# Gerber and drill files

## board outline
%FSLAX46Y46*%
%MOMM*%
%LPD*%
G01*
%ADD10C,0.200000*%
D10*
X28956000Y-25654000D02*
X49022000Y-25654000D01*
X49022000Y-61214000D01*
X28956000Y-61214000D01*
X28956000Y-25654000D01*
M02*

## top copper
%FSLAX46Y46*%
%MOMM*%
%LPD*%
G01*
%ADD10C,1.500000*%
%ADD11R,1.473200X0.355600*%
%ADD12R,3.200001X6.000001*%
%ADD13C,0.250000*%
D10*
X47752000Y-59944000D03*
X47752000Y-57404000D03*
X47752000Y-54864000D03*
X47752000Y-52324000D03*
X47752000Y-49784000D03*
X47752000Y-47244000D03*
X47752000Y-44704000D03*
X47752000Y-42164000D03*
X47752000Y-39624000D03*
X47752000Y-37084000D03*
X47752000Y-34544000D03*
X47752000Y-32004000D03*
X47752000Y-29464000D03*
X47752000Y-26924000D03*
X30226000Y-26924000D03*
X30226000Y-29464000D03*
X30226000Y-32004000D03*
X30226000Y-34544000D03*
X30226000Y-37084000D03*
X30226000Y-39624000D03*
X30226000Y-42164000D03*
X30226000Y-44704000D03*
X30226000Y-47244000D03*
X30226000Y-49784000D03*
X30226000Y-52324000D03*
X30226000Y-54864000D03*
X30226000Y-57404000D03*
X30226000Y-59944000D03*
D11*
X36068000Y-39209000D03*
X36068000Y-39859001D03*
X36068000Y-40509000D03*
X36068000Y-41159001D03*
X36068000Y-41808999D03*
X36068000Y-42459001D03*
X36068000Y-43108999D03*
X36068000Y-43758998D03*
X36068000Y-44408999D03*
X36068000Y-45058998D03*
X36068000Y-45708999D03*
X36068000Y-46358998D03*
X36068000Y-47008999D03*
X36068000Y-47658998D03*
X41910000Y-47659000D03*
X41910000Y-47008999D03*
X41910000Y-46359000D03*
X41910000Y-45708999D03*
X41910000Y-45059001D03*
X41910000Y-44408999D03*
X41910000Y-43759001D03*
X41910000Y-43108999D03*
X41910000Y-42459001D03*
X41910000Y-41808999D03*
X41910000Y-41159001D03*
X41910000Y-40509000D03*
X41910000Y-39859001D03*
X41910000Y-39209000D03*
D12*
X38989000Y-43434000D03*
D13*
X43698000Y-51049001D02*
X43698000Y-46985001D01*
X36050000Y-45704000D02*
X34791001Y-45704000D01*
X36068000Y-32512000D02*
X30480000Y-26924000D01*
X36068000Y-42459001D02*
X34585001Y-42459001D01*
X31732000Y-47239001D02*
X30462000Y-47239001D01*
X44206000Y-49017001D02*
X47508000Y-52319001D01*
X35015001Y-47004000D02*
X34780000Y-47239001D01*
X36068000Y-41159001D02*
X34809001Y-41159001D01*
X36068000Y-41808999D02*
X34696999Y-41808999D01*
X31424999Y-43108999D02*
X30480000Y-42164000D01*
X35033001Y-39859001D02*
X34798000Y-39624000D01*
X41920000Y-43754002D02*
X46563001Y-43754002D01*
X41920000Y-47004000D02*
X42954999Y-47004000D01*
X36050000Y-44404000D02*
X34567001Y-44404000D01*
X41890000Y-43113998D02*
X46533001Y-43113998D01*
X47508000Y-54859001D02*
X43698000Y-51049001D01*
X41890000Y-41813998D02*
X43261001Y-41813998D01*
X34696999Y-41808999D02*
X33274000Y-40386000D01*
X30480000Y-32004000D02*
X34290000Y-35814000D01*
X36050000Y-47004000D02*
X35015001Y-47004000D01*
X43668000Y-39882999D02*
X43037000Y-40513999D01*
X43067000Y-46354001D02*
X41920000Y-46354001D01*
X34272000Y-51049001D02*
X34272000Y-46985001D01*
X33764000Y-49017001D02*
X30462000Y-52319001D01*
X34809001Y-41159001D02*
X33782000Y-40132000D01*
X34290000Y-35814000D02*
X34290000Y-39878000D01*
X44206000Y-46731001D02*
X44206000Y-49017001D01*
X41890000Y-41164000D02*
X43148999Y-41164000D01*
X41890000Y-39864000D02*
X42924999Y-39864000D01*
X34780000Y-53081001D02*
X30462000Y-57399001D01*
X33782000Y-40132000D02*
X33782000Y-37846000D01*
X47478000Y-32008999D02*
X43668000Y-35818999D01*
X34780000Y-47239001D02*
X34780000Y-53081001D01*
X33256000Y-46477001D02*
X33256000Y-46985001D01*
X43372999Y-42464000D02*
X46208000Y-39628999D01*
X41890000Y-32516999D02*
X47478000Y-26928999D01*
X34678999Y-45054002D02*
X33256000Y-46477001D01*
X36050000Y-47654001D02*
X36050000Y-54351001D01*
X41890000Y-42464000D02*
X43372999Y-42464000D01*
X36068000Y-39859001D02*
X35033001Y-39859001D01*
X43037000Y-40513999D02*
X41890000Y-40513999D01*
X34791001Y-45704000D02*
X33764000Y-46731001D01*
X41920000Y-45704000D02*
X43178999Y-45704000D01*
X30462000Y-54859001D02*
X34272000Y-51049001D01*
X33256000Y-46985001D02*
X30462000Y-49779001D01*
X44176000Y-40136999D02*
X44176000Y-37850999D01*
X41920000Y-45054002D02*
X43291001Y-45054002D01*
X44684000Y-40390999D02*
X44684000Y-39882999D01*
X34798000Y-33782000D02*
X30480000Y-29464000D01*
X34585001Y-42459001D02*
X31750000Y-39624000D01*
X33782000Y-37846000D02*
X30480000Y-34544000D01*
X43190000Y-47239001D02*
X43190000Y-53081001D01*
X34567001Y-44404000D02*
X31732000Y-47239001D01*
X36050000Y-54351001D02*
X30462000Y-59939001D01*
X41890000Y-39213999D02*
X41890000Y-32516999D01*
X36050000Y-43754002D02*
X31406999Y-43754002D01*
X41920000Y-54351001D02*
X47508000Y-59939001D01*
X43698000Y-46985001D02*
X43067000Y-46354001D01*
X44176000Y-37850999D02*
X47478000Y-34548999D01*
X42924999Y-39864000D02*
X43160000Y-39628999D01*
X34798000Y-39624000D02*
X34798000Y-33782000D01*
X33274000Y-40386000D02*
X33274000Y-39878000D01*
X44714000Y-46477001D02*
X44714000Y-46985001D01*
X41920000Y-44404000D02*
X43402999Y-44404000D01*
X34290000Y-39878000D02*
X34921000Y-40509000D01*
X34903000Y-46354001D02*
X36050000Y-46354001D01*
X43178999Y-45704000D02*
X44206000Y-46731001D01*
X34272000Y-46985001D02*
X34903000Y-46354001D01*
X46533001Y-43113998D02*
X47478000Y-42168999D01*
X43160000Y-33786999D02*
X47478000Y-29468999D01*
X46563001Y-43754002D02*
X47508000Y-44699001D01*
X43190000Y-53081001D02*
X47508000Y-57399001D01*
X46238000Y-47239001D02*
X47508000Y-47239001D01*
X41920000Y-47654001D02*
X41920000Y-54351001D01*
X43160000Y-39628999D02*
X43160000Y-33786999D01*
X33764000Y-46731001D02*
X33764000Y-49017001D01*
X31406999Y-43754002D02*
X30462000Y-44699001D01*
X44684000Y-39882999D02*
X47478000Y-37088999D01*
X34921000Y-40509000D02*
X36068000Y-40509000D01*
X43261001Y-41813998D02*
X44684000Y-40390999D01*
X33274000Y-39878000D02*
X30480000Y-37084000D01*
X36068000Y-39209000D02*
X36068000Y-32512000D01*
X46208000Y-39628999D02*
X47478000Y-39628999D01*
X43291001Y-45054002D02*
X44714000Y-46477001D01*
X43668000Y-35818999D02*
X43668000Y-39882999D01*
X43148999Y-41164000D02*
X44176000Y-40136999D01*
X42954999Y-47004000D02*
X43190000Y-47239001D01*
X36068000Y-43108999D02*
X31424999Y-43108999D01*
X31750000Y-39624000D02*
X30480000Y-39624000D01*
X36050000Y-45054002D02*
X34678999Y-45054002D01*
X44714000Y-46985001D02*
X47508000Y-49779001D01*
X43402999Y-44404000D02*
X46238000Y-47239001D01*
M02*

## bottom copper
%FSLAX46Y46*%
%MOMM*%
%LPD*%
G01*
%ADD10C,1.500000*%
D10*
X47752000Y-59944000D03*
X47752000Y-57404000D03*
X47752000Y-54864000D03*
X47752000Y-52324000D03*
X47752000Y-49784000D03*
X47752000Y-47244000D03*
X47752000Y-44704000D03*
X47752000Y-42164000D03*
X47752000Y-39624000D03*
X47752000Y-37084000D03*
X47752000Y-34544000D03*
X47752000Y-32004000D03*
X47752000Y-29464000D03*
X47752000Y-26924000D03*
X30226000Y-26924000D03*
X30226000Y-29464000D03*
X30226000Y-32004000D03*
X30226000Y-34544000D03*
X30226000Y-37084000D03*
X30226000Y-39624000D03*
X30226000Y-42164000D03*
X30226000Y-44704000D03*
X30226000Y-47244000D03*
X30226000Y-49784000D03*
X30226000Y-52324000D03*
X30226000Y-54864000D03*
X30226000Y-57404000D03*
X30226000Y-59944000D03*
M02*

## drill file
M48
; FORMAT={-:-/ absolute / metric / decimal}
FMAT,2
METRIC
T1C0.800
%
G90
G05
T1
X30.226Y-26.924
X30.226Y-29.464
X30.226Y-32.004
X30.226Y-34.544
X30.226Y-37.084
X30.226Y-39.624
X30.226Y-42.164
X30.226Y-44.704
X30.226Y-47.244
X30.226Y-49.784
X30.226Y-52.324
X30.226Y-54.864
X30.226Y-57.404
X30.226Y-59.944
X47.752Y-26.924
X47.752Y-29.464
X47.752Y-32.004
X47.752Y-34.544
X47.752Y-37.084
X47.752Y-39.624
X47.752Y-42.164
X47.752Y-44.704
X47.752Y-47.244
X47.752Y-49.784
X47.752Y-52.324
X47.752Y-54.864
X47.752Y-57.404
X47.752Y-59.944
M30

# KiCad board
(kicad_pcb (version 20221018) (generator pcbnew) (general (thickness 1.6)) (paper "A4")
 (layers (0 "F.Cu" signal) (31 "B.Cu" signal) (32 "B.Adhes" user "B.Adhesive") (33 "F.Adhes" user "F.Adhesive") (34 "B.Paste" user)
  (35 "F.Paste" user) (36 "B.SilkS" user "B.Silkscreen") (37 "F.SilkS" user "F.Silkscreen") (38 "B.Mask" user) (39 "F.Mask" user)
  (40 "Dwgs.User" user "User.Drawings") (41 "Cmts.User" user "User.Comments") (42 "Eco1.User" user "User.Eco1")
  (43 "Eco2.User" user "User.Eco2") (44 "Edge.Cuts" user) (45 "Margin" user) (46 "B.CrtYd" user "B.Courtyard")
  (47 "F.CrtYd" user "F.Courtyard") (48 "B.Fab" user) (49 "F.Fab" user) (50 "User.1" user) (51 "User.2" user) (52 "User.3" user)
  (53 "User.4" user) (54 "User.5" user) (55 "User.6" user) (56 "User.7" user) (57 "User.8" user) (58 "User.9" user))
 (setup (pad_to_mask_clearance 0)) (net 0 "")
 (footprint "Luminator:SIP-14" (layer "F.Cu") (at 47.752 43.434 90)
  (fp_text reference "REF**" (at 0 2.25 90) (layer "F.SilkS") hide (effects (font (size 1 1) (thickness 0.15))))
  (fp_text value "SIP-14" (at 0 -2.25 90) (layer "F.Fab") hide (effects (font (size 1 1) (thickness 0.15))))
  (pad "1" thru_hole circle (at -16.51 0 90) (size 1.5 1.5) (drill 0.8) (layers "*.Cu" "*.Mask"))
  (pad "2" thru_hole circle (at -13.97 0 90) (size 1.5 1.5) (drill 0.8) (layers "*.Cu" "*.Mask"))
  (pad "3" thru_hole circle (at -11.43 0 90) (size 1.5 1.5) (drill 0.8) (layers "*.Cu" "*.Mask"))
  (pad "4" thru_hole circle (at -8.89 0 90) (size 1.5 1.5) (drill 0.8) (layers "*.Cu" "*.Mask"))
  (pad "5" thru_hole circle (at -6.35 0 90) (size 1.5 1.5) (drill 0.8) (layers "*.Cu" "*.Mask"))
  (pad "6" thru_hole circle (at -3.81 0 90) (size 1.5 1.5) (drill 0.8) (layers "*.Cu" "*.Mask"))
  (pad "7" thru_hole circle (at -1.27 0 90) (size 1.5 1.5) (drill 0.8) (layers "*.Cu" "*.Mask"))
  (pad "8" thru_hole circle (at 1.27 0 90) (size 1.5 1.5) (drill 0.8) (layers "*.Cu" "*.Mask"))
  (pad "9" thru_hole circle (at 3.81 0 90) (size 1.5 1.5) (drill 0.8) (layers "*.Cu" "*.Mask"))
  (pad "10" thru_hole circle (at 6.35 0 90) (size 1.5 1.5) (drill 0.8) (layers "*.Cu" "*.Mask"))
  (pad "11" thru_hole circle (at 8.89 0 90) (size 1.5 1.5) (drill 0.8) (layers "*.Cu" "*.Mask"))
  (pad "12" thru_hole circle (at 11.43 0 90) (size 1.5 1.5) (drill 0.8) (layers "*.Cu" "*.Mask"))
  (pad "13" thru_hole circle (at 13.97 0 90) (size 1.5 1.5) (drill 0.8) (layers "*.Cu" "*.Mask"))
  (pad "14" thru_hole circle (at 16.51 0 90) (size 1.5 1.5) (drill 0.8) (layers "*.Cu" "*.Mask")))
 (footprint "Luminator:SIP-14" (layer "F.Cu") (at 30.226 43.434 -90)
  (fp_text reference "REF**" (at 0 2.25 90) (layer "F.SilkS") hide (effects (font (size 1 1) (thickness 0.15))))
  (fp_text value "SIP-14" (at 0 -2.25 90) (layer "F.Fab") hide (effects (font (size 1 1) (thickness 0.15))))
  (pad "1" thru_hole circle (at -16.51 0 270) (size 1.5 1.5) (drill 0.8) (layers "*.Cu" "*.Mask"))
  (pad "2" thru_hole circle (at -13.97 0 270) (size 1.5 1.5) (drill 0.8) (layers "*.Cu" "*.Mask"))
  (pad "3" thru_hole circle (at -11.43 0 270) (size 1.5 1.5) (drill 0.8) (layers "*.Cu" "*.Mask"))
  (pad "4" thru_hole circle (at -8.89 0 270) (size 1.5 1.5) (drill 0.8) (layers "*.Cu" "*.Mask"))
  (pad "5" thru_hole circle (at -6.35 0 270) (size 1.5 1.5) (drill 0.8) (layers "*.Cu" "*.Mask"))
  (pad "6" thru_hole circle (at -3.81 0 270) (size 1.5 1.5) (drill 0.8) (layers "*.Cu" "*.Mask"))
  (pad "7" thru_hole circle (at -1.27 0 270) (size 1.5 1.5) (drill 0.8) (layers "*.Cu" "*.Mask"))
  (pad "8" thru_hole circle (at 1.27 0 270) (size 1.5 1.5) (drill 0.8) (layers "*.Cu" "*.Mask"))
  (pad "9" thru_hole circle (at 3.81 0 270) (size 1.5 1.5) (drill 0.8) (layers "*.Cu" "*.Mask"))
  (pad "10" thru_hole circle (at 6.35 0 270) (size 1.5 1.5) (drill 0.8) (layers "*.Cu" "*.Mask"))
  (pad "11" thru_hole circle (at 8.89 0 270) (size 1.5 1.5) (drill 0.8) (layers "*.Cu" "*.Mask"))
  (pad "12" thru_hole circle (at 11.43 0 270) (size 1.5 1.5) (drill 0.8) (layers "*.Cu" "*.Mask"))
  (pad "13" thru_hole circle (at 13.97 0 270) (size 1.5 1.5) (drill 0.8) (layers "*.Cu" "*.Mask"))
  (pad "14" thru_hole circle (at 16.51 0 270) (size 1.5 1.5) (drill 0.8) (layers "*.Cu" "*.Mask")))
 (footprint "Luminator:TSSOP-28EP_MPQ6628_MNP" (layer "F.Cu") (at 38.989 43.434)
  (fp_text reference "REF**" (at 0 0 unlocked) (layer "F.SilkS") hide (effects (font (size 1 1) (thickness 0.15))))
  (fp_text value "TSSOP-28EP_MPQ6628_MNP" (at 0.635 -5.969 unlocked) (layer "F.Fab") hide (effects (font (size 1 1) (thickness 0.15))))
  (pad "1" smd rect (at -2.921 -4.225) (size 1.4732 0.3556) (layers "F.Cu" "F.Paste" "F.Mask"))
  (pad "2" smd rect (at -2.921 -3.574999) (size 1.4732 0.3556) (layers "F.Cu" "F.Paste" "F.Mask"))
  (pad "3" smd rect (at -2.921 -2.925) (size 1.4732 0.3556) (layers "F.Cu" "F.Paste" "F.Mask"))
  (pad "4" smd rect (at -2.921 -2.274999) (size 1.4732 0.3556) (layers "F.Cu" "F.Paste" "F.Mask"))
  (pad "5" smd rect (at -2.921 -1.625001) (size 1.4732 0.3556) (layers "F.Cu" "F.Paste" "F.Mask"))
  (pad "6" smd rect (at -2.921 -0.974999) (size 1.4732 0.3556) (layers "F.Cu" "F.Paste" "F.Mask"))
  (pad "7" smd rect (at -2.921 -0.325001) (size 1.4732 0.3556) (layers "F.Cu" "F.Paste" "F.Mask"))
  (pad "8" smd rect (at -2.921 0.324998) (size 1.4732 0.3556) (layers "F.Cu" "F.Paste" "F.Mask"))
  (pad "9" smd rect (at -2.921 0.974999) (size 1.4732 0.3556) (layers "F.Cu" "F.Paste" "F.Mask"))
  (pad "10" smd rect (at -2.921 1.624998) (size 1.4732 0.3556) (layers "F.Cu" "F.Paste" "F.Mask"))
  (pad "11" smd rect (at -2.921 2.274999) (size 1.4732 0.3556) (layers "F.Cu" "F.Paste" "F.Mask"))
  (pad "12" smd rect (at -2.921 2.924998) (size 1.4732 0.3556) (layers "F.Cu" "F.Paste" "F.Mask"))
  (pad "13" smd rect (at -2.921 3.574999) (size 1.4732 0.3556) (layers "F.Cu" "F.Paste" "F.Mask"))
  (pad "14" smd rect (at -2.921 4.224998) (size 1.4732 0.3556) (layers "F.Cu" "F.Paste" "F.Mask"))
  (pad "15" smd rect (at 2.921 4.225) (size 1.4732 0.3556) (layers "F.Cu" "F.Paste" "F.Mask"))
  (pad "16" smd rect (at 2.921 3.574999) (size 1.4732 0.3556) (layers "F.Cu" "F.Paste" "F.Mask"))
  (pad "17" smd rect (at 2.921 2.925) (size 1.4732 0.3556) (layers "F.Cu" "F.Paste" "F.Mask"))
  (pad "18" smd rect (at 2.921 2.274999) (size 1.4732 0.3556) (layers "F.Cu" "F.Paste" "F.Mask"))
  (pad "19" smd rect (at 2.921 1.625001) (size 1.4732 0.3556) (layers "F.Cu" "F.Paste" "F.Mask"))
  (pad "20" smd rect (at 2.921 0.974999) (size 1.4732 0.3556) (layers "F.Cu" "F.Paste" "F.Mask"))
  (pad "21" smd rect (at 2.921 0.325001) (size 1.4732 0.3556) (layers "F.Cu" "F.Paste" "F.Mask"))
  (pad "22" smd rect (at 2.921 -0.325001) (size 1.4732 0.3556) (layers "F.Cu" "F.Paste" "F.Mask"))
  (pad "23" smd rect (at 2.921 -0.974999) (size 1.4732 0.3556) (layers "F.Cu" "F.Paste" "F.Mask"))
  (pad "24" smd rect (at 2.921 -1.625001) (size 1.4732 0.3556) (layers "F.Cu" "F.Paste" "F.Mask"))
  (pad "25" smd rect (at 2.921 -2.274999) (size 1.4732 0.3556) (layers "F.Cu" "F.Paste" "F.Mask"))
  (pad "26" smd rect (at 2.921 -2.925) (size 1.4732 0.3556) (layers "F.Cu" "F.Paste" "F.Mask"))
  (pad "27" smd rect (at 2.921 -3.574999) (size 1.4732 0.3556) (layers "F.Cu" "F.Paste" "F.Mask"))
  (pad "28" smd rect (at 2.921 -4.225) (size 1.4732 0.3556) (layers "F.Cu" "F.Paste" "F.Mask"))
  (pad "29" smd rect (at 0 0) (size 3.200001 6.000001) (layers "F.Cu" "F.Mask")))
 (gr_rect (start 28.956 25.654) (end 49.022 61.214) (stroke (width 0.2) (type default)) (fill none) (layer "Edge.Cuts"))
 (segment (start 43.698 51.049001) (end 43.698 46.985001) (width 0.25) (layer "F.Cu") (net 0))
 (segment (start 36.05 45.704) (end 34.791001 45.704) (width 0.25) (layer "F.Cu") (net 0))
 (segment (start 36.068 32.512) (end 30.48 26.924) (width 0.25) (layer "F.Cu") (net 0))
 (segment (start 36.068 42.459001) (end 34.585001 42.459001) (width 0.25) (layer "F.Cu") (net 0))
 (segment (start 31.732 47.239001) (end 30.462 47.239001) (width 0.25) (layer "F.Cu") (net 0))
 (segment (start 44.206 49.017001) (end 47.508 52.319001) (width 0.25) (layer "F.Cu") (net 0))
 (segment (start 35.015001 47.004) (end 34.78 47.239001) (width 0.25) (layer "F.Cu") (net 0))
 (segment (start 36.068 41.159001) (end 34.809001 41.159001) (width 0.25) (layer "F.Cu") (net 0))
 (segment (start 36.068 41.808999) (end 34.696999 41.808999) (width 0.25) (layer "F.Cu") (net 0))
 (segment (start 31.424999 43.108999) (end 30.48 42.164) (width 0.25) (layer "F.Cu") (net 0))
 (segment (start 35.033001 39.859001) (end 34.798 39.624) (width 0.25) (layer "F.Cu") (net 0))
 (segment (start 41.92 43.754002) (end 46.563001 43.754002) (width 0.25) (layer "F.Cu") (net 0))
 (segment (start 41.92 47.004) (end 42.954999 47.004) (width 0.25) (layer "F.Cu") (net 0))
 (segment (start 36.05 44.404) (end 34.567001 44.404) (width 0.25) (layer "F.Cu") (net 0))
 (segment (start 41.89 43.113998) (end 46.533001 43.113998) (width 0.25) (layer "F.Cu") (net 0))
 (segment (start 47.508 54.859001) (end 43.698 51.049001) (width 0.25) (layer "F.Cu") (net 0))
 (segment (start 41.89 41.813998) (end 43.261001 41.813998) (width 0.25) (layer "F.Cu") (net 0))
 (segment (start 34.696999 41.808999) (end 33.274 40.386) (width 0.25) (layer "F.Cu") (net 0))
 (segment (start 30.48 32.004) (end 34.29 35.814) (width 0.25) (layer "F.Cu") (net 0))
 (segment (start 36.05 47.004) (end 35.015001 47.004) (width 0.25) (layer "F.Cu") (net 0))
 (segment (start 43.668 39.882999) (end 43.037 40.513999) (width 0.25) (layer "F.Cu") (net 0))
 (segment (start 43.067 46.354001) (end 41.92 46.354001) (width 0.25) (layer "F.Cu") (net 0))
 (segment (start 34.272 51.049001) (end 34.272 46.985001) (width 0.25) (layer "F.Cu") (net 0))
 (segment (start 33.764 49.017001) (end 30.462 52.319001) (width 0.25) (layer "F.Cu") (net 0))
 (segment (start 34.809001 41.159001) (end 33.782 40.132) (width 0.25) (layer "F.Cu") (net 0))
 (segment (start 34.29 35.814) (end 34.29 39.878) (width 0.25) (layer "F.Cu") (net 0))
 (segment (start 44.206 46.731001) (end 44.206 49.017001) (width 0.25) (layer "F.Cu") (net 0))
 (segment (start 41.89 41.164) (end 43.148999 41.164) (width 0.25) (layer "F.Cu") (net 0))
 (segment (start 41.89 39.864) (end 42.924999 39.864) (width 0.25) (layer "F.Cu") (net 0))
 (segment (start 34.78 53.081001) (end 30.462 57.399001) (width 0.25) (layer "F.Cu") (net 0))
 (segment (start 33.782 40.132) (end 33.782 37.846) (width 0.25) (layer "F.Cu") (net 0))
 (segment (start 47.478 32.008999) (end 43.668 35.818999) (width 0.25) (layer "F.Cu") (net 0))
 (segment (start 34.78 47.239001) (end 34.78 53.081001) (width 0.25) (layer "F.Cu") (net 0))
 (segment (start 33.256 46.477001) (end 33.256 46.985001) (width 0.25) (layer "F.Cu") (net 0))
 (segment (start 43.372999 42.464) (end 46.208 39.628999) (width 0.25) (layer "F.Cu") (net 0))
 (segment (start 41.89 32.516999) (end 47.478 26.928999) (width 0.25) (layer "F.Cu") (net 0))
 (segment (start 34.678999 45.054002) (end 33.256 46.477001) (width 0.25) (layer "F.Cu") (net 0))
 (segment (start 36.05 47.654001) (end 36.05 54.351001) (width 0.25) (layer "F.Cu") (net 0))
 (segment (start 41.89 42.464) (end 43.372999 42.464) (width 0.25) (layer "F.Cu") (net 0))
 (segment (start 36.068 39.859001) (end 35.033001 39.859001) (width 0.25) (layer "F.Cu") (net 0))
 (segment (start 43.037 40.513999) (end 41.89 40.513999) (width 0.25) (layer "F.Cu") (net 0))
 (segment (start 34.791001 45.704) (end 33.764 46.731001) (width 0.25) (layer "F.Cu") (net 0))
 (segment (start 41.92 45.704) (end 43.178999 45.704) (width 0.25) (layer "F.Cu") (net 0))
 (segment (start 30.462 54.859001) (end 34.272 51.049001) (width 0.25) (layer "F.Cu") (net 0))
 (segment (start 33.256 46.985001) (end 30.462 49.779001) (width 0.25) (layer "F.Cu") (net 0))
 (segment (start 44.176 40.136999) (end 44.176 37.850999) (width 0.25) (layer "F.Cu") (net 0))
 (segment (start 41.92 45.054002) (end 43.291001 45.054002) (width 0.25) (layer "F.Cu") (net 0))
 (segment (start 44.684 40.390999) (end 44.684 39.882999) (width 0.25) (layer "F.Cu") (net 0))
 (segment (start 34.798 33.782) (end 30.48 29.464) (width 0.25) (layer "F.Cu") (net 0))
 (segment (start 34.585001 42.459001) (end 31.75 39.624) (width 0.25) (layer "F.Cu") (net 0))
 (segment (start 33.782 37.846) (end 30.48 34.544) (width 0.25) (layer "F.Cu") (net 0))
 (segment (start 43.19 47.239001) (end 43.19 53.081001) (width 0.25) (layer "F.Cu") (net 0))
 (segment (start 34.567001 44.404) (end 31.732 47.239001) (width 0.25) (layer "F.Cu") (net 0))
 (segment (start 36.05 54.351001) (end 30.462 59.939001) (width 0.25) (layer "F.Cu") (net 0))
 (segment (start 41.89 39.213999) (end 41.89 32.516999) (width 0.25) (layer "F.Cu") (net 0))
 (segment (start 36.05 43.754002) (end 31.406999 43.754002) (width 0.25) (layer "F.Cu") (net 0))
 (segment (start 41.92 54.351001) (end 47.508 59.939001) (width 0.25) (layer "F.Cu") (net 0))
 (segment (start 43.698 46.985001) (end 43.067 46.354001) (width 0.25) (layer "F.Cu") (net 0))
 (segment (start 44.176 37.850999) (end 47.478 34.548999) (width 0.25) (layer "F.Cu") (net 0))
 (segment (start 42.924999 39.864) (end 43.16 39.628999) (width 0.25) (layer "F.Cu") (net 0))
 (segment (start 34.798 39.624) (end 34.798 33.782) (width 0.25) (layer "F.Cu") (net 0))
 (segment (start 33.274 40.386) (end 33.274 39.878) (width 0.25) (layer "F.Cu") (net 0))
 (segment (start 44.714 46.477001) (end 44.714 46.985001) (width 0.25) (layer "F.Cu") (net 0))
 (segment (start 41.92 44.404) (end 43.402999 44.404) (width 0.25) (layer "F.Cu") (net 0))
 (segment (start 34.29 39.878) (end 34.921 40.509) (width 0.25) (layer "F.Cu") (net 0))
 (segment (start 34.903 46.354001) (end 36.05 46.354001) (width 0.25) (layer "F.Cu") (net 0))
 (segment (start 43.178999 45.704) (end 44.206 46.731001) (width 0.25) (layer "F.Cu") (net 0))
 (segment (start 34.272 46.985001) (end 34.903 46.354001) (width 0.25) (layer "F.Cu") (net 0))
 (segment (start 46.533001 43.113998) (end 47.478 42.168999) (width 0.25) (layer "F.Cu") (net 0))
 (segment (start 43.16 33.786999) (end 47.478 29.468999) (width 0.25) (layer "F.Cu") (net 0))
 (segment (start 46.563001 43.754002) (end 47.508 44.699001) (width 0.25) (layer "F.Cu") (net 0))
 (segment (start 43.19 53.081001) (end 47.508 57.399001) (width 0.25) (layer "F.Cu") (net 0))
 (segment (start 46.238 47.239001) (end 47.508 47.239001) (width 0.25) (layer "F.Cu") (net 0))
 (segment (start 41.92 47.654001) (end 41.92 54.351001) (width 0.25) (layer "F.Cu") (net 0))
 (segment (start 43.16 39.628999) (end 43.16 33.786999) (width 0.25) (layer "F.Cu") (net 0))
 (segment (start 33.764 46.731001) (end 33.764 49.017001) (width 0.25) (layer "F.Cu") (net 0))
 (segment (start 31.406999 43.754002) (end 30.462 44.699001) (width 0.25) (layer "F.Cu") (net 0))
 (segment (start 44.684 39.882999) (end 47.478 37.088999) (width 0.25) (layer "F.Cu") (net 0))
 (segment (start 34.921 40.509) (end 36.068 40.509) (width 0.25) (layer "F.Cu") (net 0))
 (segment (start 43.261001 41.813998) (end 44.684 40.390999) (width 0.25) (layer "F.Cu") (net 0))
 (segment (start 33.274 39.878) (end 30.48 37.084) (width 0.25) (layer "F.Cu") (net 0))
 (segment (start 36.068 39.209) (end 36.068 32.512) (width 0.25) (layer "F.Cu") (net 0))
 (segment (start 46.208 39.628999) (end 47.478 39.628999) (width 0.25) (layer "F.Cu") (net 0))
 (segment (start 43.291001 45.054002) (end 44.714 46.477001) (width 0.25) (layer "F.Cu") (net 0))
 (segment (start 43.668 35.818999) (end 43.668 39.882999) (width 0.25) (layer "F.Cu") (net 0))
 (segment (start 43.148999 41.164) (end 44.176 40.136999) (width 0.25) (layer "F.Cu") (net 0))
 (segment (start 42.954999 47.004) (end 43.19 47.239001) (width 0.25) (layer "F.Cu") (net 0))
 (segment (start 36.068 43.108999) (end 31.424999 43.108999) (width 0.25) (layer "F.Cu") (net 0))
 (segment (start 31.75 39.624) (end 30.48 39.624) (width 0.25) (layer "F.Cu") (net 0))
 (segment (start 36.05 45.054002) (end 34.678999 45.054002) (width 0.25) (layer "F.Cu") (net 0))
 (segment (start 44.714 46.985001) (end 47.508 49.779001) (width 0.25) (layer "F.Cu") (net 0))
 (segment (start 43.402999 44.404) (end 46.238 47.239001) (width 0.25) (layer "F.Cu") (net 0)))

